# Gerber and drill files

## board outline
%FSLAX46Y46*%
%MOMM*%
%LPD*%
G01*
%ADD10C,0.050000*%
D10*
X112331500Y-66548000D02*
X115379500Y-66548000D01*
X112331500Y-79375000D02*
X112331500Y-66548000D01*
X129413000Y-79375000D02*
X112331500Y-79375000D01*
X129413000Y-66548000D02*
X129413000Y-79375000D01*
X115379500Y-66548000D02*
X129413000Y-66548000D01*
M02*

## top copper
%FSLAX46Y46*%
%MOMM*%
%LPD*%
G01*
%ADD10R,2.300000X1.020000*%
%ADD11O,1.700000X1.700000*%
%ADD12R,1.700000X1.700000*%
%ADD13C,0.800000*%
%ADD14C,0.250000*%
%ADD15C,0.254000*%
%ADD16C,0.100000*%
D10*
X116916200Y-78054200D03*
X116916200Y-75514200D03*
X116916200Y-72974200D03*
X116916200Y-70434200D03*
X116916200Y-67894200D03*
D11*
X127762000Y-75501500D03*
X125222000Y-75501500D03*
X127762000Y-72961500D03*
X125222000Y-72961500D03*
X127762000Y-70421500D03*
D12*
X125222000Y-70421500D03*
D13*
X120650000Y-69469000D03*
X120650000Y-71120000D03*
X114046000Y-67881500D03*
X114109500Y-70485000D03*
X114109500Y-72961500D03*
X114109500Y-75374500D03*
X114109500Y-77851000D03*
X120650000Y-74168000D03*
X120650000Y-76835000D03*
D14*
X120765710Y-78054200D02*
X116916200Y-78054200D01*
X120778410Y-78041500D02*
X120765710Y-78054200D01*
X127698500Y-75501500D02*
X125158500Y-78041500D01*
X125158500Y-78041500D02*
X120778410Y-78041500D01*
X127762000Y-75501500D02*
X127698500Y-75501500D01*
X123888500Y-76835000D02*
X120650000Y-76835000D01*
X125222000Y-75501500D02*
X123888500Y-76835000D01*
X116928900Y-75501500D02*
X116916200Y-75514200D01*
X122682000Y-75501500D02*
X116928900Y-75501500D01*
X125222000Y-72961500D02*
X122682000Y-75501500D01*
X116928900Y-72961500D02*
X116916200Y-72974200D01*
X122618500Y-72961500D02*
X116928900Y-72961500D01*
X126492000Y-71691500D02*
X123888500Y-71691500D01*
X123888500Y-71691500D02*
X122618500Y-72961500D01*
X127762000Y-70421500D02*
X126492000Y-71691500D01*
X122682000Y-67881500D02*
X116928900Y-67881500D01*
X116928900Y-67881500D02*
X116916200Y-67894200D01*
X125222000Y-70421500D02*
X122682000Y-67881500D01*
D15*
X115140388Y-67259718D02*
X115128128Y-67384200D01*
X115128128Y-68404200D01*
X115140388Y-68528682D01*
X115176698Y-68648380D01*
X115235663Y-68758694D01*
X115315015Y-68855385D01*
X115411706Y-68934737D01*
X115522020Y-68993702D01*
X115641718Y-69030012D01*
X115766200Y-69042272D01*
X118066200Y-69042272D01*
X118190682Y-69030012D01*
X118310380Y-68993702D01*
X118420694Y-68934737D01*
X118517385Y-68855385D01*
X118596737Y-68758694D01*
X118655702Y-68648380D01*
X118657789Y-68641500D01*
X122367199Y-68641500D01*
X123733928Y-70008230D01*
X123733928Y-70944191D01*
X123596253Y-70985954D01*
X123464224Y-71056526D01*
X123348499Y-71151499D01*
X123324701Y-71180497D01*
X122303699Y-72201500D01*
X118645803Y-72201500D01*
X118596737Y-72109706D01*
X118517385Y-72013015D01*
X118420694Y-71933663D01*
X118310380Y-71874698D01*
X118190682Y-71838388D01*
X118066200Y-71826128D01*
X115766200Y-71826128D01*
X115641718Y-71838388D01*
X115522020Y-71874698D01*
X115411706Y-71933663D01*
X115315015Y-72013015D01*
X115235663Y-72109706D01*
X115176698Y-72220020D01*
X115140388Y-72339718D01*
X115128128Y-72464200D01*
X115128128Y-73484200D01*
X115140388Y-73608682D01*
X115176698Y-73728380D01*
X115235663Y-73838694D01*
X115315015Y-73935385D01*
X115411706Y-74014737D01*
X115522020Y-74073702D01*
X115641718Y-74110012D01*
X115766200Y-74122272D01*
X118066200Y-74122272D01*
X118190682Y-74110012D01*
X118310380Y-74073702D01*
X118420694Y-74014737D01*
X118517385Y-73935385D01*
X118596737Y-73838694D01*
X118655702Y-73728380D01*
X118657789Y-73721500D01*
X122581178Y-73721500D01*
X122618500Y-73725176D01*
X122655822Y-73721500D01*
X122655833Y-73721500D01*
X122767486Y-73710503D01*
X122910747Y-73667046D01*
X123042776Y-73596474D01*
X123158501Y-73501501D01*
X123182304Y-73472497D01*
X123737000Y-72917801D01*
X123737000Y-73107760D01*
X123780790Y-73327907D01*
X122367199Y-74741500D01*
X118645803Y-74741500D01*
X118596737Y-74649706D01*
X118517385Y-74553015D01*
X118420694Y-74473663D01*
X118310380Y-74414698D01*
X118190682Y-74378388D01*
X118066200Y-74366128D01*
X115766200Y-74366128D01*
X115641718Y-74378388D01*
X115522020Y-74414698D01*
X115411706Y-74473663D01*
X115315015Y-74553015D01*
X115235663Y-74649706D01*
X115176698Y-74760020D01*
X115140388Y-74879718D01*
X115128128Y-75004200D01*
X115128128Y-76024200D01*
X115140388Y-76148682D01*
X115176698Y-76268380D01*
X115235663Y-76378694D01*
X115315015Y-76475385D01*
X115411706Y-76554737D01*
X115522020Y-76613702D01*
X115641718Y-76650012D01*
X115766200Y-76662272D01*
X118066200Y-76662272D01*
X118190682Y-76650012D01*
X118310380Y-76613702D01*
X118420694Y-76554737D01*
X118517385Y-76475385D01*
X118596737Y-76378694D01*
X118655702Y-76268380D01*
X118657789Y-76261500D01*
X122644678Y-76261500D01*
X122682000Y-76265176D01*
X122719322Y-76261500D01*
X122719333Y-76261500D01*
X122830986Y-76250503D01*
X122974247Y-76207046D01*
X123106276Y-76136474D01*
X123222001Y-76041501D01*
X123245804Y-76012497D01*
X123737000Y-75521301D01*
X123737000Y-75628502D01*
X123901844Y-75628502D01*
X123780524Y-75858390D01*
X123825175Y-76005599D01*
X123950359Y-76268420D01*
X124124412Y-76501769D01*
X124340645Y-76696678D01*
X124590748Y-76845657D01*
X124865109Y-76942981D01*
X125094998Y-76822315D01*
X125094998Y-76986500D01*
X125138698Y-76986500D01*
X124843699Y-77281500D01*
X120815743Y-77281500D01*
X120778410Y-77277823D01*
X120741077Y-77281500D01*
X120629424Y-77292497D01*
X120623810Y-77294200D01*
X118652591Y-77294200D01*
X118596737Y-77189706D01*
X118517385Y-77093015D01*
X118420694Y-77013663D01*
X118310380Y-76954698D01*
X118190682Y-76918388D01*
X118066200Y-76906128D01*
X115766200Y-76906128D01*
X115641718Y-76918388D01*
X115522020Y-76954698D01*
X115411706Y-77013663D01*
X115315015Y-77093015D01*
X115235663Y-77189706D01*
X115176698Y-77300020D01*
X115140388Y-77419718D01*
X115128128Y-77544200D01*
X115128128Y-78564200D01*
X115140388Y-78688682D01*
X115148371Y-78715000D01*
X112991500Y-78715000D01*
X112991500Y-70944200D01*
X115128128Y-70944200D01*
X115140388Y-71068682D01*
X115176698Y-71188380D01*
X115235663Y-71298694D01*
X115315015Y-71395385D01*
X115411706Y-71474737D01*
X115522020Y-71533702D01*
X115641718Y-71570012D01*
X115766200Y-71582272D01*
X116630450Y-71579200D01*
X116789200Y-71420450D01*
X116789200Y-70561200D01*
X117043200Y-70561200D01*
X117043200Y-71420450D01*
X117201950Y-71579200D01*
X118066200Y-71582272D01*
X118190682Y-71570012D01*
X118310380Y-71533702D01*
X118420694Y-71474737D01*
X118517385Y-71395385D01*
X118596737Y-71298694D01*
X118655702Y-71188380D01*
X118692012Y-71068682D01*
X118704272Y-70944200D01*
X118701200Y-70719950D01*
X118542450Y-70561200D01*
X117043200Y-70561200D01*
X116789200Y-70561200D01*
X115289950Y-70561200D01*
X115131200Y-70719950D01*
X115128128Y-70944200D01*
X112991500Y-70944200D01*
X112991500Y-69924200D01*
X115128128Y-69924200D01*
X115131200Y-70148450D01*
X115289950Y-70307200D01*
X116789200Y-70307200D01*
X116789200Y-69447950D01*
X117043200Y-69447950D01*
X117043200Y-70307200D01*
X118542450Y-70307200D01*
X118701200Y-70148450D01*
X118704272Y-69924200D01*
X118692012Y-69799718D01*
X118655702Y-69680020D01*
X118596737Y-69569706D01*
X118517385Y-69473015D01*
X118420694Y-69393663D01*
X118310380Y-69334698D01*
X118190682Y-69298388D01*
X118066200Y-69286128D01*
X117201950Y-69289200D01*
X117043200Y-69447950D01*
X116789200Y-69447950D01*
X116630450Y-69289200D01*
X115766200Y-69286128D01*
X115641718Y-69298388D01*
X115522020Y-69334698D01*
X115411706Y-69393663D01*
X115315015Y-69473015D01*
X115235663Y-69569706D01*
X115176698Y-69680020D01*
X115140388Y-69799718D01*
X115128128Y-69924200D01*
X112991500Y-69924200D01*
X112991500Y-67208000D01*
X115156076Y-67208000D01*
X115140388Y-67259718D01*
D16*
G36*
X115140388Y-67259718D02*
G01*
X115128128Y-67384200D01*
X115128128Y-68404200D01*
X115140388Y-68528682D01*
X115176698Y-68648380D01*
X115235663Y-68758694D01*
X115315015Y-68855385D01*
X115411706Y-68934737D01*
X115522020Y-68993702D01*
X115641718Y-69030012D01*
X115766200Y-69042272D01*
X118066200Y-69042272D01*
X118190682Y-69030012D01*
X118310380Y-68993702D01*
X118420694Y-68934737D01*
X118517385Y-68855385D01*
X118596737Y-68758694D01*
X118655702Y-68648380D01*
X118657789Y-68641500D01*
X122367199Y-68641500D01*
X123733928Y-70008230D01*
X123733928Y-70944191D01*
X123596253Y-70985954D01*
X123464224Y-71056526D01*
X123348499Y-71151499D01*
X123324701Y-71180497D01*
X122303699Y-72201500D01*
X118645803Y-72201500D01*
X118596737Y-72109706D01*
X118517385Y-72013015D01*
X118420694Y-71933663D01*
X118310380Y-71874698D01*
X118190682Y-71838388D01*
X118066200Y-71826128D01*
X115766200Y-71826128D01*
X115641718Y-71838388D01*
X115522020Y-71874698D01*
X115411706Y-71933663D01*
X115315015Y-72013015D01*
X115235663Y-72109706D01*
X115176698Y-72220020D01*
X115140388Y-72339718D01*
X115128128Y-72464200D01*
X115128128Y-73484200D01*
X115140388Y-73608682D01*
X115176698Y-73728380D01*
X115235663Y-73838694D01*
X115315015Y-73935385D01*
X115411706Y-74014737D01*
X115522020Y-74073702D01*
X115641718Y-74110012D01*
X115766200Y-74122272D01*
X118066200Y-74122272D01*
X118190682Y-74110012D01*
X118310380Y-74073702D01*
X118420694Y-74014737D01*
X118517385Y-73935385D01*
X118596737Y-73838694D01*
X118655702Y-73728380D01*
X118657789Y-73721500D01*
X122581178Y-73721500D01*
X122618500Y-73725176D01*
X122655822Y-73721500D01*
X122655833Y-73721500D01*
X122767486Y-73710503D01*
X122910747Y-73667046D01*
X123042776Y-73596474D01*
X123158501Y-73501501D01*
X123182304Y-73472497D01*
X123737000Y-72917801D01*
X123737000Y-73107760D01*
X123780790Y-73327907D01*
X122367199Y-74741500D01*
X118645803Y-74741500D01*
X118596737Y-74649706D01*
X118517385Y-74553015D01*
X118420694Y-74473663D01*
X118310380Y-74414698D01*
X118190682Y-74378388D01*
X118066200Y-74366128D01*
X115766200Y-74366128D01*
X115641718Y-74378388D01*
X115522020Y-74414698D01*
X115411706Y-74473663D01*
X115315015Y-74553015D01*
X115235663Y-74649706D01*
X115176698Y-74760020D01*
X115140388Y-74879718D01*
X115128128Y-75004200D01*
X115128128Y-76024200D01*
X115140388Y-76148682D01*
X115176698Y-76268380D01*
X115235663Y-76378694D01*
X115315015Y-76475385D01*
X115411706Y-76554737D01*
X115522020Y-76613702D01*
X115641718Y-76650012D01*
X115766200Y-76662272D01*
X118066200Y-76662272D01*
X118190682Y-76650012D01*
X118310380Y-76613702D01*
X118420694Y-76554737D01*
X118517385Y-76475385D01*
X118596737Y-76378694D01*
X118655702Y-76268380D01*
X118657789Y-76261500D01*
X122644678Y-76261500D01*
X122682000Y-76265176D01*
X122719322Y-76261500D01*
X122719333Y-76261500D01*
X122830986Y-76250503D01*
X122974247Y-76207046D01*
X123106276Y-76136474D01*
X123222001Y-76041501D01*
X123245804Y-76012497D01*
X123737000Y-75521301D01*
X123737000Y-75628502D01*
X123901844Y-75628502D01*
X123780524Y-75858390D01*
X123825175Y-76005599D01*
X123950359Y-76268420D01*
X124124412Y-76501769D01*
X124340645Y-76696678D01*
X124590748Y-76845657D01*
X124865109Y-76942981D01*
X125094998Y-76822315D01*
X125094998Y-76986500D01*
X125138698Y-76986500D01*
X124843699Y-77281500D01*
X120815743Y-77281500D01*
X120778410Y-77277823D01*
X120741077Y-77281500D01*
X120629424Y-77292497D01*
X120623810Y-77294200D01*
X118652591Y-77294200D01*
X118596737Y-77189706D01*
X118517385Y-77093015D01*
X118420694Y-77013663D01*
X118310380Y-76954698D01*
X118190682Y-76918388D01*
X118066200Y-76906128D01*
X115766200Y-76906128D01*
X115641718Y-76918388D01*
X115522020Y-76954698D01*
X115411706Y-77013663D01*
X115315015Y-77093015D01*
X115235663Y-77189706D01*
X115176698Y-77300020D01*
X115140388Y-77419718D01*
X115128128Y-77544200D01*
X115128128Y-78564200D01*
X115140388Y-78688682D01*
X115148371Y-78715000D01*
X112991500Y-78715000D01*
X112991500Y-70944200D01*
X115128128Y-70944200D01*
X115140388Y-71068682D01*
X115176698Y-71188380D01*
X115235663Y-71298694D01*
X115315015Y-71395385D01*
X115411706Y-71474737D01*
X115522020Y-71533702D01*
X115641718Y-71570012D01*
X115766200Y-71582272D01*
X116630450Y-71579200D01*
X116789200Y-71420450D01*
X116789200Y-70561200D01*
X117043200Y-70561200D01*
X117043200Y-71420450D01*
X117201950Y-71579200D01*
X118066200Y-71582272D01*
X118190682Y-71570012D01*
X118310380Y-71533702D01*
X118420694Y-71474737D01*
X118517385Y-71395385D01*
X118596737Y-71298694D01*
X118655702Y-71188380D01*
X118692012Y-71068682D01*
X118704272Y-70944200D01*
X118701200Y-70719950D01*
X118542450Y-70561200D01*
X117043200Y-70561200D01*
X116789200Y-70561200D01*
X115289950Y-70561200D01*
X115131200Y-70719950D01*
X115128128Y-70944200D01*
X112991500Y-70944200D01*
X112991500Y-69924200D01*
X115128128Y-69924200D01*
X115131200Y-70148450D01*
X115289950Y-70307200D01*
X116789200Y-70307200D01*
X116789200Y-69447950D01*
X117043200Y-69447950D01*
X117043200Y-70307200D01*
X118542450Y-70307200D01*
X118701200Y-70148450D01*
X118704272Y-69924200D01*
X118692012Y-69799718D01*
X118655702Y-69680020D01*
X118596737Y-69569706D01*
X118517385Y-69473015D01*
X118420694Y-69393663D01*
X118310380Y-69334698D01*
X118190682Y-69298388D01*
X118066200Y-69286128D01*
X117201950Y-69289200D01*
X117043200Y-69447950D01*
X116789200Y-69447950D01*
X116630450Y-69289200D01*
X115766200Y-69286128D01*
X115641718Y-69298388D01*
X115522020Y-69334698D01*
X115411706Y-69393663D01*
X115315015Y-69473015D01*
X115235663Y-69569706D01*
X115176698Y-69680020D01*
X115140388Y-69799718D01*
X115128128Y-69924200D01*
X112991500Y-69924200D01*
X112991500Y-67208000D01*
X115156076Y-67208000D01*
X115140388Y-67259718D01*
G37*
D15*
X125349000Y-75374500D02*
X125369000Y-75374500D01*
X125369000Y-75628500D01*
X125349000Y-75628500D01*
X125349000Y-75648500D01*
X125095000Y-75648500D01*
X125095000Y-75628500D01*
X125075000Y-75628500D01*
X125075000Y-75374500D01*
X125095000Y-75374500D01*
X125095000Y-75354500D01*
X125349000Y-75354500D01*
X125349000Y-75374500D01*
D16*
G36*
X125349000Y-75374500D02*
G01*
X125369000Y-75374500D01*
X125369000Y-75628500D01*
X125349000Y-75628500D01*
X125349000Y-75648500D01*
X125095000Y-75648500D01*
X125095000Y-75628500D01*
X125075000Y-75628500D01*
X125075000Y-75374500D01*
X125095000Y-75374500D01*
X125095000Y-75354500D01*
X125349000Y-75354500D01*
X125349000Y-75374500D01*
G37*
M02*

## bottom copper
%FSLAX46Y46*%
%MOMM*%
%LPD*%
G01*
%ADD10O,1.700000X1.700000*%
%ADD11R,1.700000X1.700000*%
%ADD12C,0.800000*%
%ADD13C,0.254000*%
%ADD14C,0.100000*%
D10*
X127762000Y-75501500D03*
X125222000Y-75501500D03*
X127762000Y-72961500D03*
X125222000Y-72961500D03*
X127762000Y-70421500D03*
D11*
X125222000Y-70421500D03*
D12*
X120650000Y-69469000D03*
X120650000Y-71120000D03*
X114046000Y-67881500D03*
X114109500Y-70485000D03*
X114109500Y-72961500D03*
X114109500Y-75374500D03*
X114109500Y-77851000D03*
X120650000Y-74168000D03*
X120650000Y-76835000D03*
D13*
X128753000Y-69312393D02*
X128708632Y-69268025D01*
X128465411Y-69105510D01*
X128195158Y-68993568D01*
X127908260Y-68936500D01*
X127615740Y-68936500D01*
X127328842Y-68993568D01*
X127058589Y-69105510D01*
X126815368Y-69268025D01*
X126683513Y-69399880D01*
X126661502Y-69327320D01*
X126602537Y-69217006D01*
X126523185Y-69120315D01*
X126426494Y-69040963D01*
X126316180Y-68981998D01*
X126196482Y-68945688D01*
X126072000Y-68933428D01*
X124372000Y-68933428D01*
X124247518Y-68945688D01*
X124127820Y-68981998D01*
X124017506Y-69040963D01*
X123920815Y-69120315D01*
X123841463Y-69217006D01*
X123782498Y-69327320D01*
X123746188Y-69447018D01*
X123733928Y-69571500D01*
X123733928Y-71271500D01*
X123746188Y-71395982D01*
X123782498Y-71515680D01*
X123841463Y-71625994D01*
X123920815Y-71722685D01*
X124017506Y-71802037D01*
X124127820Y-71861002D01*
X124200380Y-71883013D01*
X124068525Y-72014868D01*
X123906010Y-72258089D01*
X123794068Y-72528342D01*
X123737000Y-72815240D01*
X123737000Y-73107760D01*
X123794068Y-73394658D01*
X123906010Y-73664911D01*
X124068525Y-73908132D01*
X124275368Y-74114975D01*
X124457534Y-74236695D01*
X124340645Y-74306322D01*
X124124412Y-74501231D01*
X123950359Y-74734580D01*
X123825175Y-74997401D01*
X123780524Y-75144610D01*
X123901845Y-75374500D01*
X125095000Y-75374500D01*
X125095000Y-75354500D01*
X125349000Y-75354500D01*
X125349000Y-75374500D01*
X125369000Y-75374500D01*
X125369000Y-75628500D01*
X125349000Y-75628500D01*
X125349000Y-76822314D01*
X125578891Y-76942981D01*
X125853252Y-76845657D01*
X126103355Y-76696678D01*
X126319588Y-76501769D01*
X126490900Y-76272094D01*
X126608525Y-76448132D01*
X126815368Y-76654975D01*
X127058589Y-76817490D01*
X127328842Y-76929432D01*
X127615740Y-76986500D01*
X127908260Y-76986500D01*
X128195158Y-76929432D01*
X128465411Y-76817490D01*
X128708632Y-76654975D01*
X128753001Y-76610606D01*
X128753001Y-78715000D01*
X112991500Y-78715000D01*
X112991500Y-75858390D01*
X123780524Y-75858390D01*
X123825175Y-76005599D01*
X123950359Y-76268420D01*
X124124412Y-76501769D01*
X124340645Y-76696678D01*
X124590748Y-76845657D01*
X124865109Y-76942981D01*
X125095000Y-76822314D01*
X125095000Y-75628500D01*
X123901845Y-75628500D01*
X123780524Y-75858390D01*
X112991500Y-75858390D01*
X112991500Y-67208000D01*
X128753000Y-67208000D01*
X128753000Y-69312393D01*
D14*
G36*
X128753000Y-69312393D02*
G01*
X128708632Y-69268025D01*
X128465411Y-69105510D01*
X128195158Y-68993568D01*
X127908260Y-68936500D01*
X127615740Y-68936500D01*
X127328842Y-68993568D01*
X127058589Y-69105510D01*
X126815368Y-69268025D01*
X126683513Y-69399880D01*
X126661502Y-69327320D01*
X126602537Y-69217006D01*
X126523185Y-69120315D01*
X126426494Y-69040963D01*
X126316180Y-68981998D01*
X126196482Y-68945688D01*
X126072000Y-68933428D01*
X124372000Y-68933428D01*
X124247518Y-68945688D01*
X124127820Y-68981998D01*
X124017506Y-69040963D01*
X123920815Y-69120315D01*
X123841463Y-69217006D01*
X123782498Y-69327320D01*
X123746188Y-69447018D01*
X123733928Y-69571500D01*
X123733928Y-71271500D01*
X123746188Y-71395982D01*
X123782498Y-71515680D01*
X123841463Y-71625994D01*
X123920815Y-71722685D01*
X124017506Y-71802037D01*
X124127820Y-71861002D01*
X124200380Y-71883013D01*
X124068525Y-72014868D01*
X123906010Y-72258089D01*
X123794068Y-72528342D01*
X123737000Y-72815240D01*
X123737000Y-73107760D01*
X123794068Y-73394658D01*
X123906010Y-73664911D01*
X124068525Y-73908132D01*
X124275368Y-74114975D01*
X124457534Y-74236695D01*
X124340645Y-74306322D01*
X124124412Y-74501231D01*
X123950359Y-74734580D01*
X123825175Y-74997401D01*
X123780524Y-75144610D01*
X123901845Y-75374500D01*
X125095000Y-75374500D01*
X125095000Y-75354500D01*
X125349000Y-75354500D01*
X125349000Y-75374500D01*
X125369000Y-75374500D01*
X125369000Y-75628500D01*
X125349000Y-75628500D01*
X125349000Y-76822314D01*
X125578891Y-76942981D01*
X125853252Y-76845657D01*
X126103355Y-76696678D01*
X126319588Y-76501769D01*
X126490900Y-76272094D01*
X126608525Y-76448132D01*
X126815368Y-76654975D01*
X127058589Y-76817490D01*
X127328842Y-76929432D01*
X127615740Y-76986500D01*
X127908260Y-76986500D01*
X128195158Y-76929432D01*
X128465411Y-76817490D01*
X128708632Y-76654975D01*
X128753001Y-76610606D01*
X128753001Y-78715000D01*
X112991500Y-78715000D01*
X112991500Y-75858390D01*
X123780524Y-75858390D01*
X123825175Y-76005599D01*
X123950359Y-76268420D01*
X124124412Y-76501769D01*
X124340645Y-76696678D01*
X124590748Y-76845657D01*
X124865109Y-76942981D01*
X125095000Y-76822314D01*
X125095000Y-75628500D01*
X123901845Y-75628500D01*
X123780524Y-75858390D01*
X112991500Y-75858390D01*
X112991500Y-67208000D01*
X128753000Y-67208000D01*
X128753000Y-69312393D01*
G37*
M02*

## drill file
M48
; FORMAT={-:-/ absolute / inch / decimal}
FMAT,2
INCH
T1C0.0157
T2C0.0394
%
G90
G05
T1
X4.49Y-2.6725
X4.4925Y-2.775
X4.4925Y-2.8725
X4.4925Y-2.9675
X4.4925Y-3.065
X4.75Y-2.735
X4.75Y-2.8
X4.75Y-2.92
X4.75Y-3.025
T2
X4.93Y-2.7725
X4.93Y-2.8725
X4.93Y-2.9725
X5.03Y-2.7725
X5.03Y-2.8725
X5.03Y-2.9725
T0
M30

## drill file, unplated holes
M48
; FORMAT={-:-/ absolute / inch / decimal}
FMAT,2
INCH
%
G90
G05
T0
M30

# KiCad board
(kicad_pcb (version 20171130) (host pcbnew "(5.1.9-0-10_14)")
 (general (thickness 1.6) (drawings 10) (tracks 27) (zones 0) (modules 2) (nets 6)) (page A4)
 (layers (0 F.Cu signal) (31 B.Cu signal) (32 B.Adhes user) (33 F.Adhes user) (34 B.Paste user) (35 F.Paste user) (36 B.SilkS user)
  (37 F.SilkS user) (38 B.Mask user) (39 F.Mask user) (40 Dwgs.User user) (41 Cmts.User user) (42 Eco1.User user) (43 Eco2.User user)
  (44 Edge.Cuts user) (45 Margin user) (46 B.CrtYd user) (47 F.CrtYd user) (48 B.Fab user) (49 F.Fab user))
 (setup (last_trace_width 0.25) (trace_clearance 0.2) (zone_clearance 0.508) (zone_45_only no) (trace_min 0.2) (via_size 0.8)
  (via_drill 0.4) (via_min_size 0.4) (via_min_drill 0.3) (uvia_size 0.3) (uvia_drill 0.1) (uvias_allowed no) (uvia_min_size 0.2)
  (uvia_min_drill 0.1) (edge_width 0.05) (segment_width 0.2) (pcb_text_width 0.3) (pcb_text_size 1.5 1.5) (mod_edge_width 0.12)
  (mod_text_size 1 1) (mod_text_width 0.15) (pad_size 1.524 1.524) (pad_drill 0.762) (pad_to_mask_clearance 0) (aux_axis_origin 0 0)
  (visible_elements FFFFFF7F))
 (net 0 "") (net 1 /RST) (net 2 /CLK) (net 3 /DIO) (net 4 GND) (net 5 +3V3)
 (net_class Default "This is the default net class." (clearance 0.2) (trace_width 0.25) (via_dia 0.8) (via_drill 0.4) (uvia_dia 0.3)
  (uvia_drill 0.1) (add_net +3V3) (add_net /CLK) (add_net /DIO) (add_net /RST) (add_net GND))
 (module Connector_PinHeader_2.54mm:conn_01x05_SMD (layer F.Cu) (at 116.967 65.659)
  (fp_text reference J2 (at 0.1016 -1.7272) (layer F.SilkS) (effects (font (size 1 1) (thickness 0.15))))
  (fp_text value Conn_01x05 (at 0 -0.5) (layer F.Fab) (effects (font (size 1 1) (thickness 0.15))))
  (pad 5 smd rect (at -0.0508 12.3952 90) (size 1.02 2.3) (layers F.Cu F.Paste F.Mask) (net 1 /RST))
  (pad 4 smd rect (at -0.0508 9.8552 90) (size 1.02 2.3) (layers F.Cu F.Paste F.Mask) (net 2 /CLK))
  (pad 3 smd rect (at -0.0508 7.3152 90) (size 1.02 2.3) (layers F.Cu F.Paste F.Mask) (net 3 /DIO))
  (pad 2 smd rect (at -0.0508 4.7752 90) (size 1.02 2.3) (layers F.Cu F.Paste F.Mask) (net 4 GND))
  (pad 1 smd rect (at -0.0508 2.2352 90) (size 1.02 2.3) (layers F.Cu F.Paste F.Mask) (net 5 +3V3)))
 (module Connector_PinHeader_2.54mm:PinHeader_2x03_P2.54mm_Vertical (layer F.Cu) (at 125.222 70.4215)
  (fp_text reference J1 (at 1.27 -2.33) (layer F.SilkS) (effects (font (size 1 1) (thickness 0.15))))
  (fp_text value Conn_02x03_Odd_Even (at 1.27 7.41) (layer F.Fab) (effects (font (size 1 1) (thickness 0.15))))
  (pad 6 thru_hole oval (at 2.54 5.08) (size 1.7 1.7) (drill 1) (layers *.Cu *.Mask) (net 1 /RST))
  (pad 5 thru_hole oval (at 0 5.08) (size 1.7 1.7) (drill 1) (layers *.Cu *.Mask) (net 4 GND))
  (pad 4 thru_hole oval (at 2.54 2.54) (size 1.7 1.7) (drill 1) (layers *.Cu *.Mask))
  (pad 3 thru_hole oval (at 0 2.54) (size 1.7 1.7) (drill 1) (layers *.Cu *.Mask) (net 2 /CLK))
  (pad 2 thru_hole oval (at 2.54 0) (size 1.7 1.7) (drill 1) (layers *.Cu *.Mask) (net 3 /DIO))
  (pad 1 thru_hole rect (at 0 0) (size 1.7 1.7) (drill 1) (layers *.Cu *.Mask) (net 5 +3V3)))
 (gr_line (start 112.3315 66.548) (end 115.3795 66.548) (layer Edge.Cuts) (width 0.05))
 (gr_line (start 112.3315 79.375) (end 112.3315 66.548) (layer Edge.Cuts) (width 0.05))
 (gr_line (start 129.413 79.375) (end 112.3315 79.375) (layer Edge.Cuts) (width 0.05))
 (gr_line (start 129.413 66.548) (end 129.413 79.375) (layer Edge.Cuts) (width 0.05))
 (gr_line (start 115.3795 66.548) (end 129.413 66.548) (layer Edge.Cuts) (width 0.05))
 (segment (start 120.76571 78.0542) (end 116.9162 78.0542) (width 0.25) (layer F.Cu) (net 1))
 (segment (start 120.77841 78.0415) (end 120.76571 78.0542) (width 0.25) (layer F.Cu) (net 1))
 (segment (start 127.6985 75.5015) (end 125.1585 78.0415) (width 0.25) (layer F.Cu) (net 1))
 (segment (start 125.1585 78.0415) (end 120.77841 78.0415) (width 0.25) (layer F.Cu) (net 1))
 (segment (start 127.762 75.5015) (end 127.6985 75.5015) (width 0.25) (layer F.Cu) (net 1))
 (via (at 120.65 69.469) (size 0.8) (drill 0.4) (layers F.Cu B.Cu) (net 4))
 (via (at 120.65 71.12) (size 0.8) (drill 0.4) (layers F.Cu B.Cu) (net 4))
 (via (at 114.046 67.8815) (size 0.8) (drill 0.4) (layers F.Cu B.Cu) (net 4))
 (via (at 114.1095 70.485) (size 0.8) (drill 0.4) (layers F.Cu B.Cu) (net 4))
 (via (at 114.1095 72.9615) (size 0.8) (drill 0.4) (layers F.Cu B.Cu) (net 4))
 (via (at 114.1095 75.3745) (size 0.8) (drill 0.4) (layers F.Cu B.Cu) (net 4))
 (via (at 114.1095 77.851) (size 0.8) (drill 0.4) (layers F.Cu B.Cu) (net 4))
 (via (at 120.65 74.168) (size 0.8) (drill 0.4) (layers F.Cu B.Cu) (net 4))
 (via (at 120.65 76.835) (size 0.8) (drill 0.4) (layers F.Cu B.Cu) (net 4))
 (segment (start 123.8885 76.835) (end 120.65 76.835) (width 0.25) (layer F.Cu) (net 4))
 (segment (start 125.222 75.5015) (end 123.8885 76.835) (width 0.25) (layer F.Cu) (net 4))
 (segment (start 116.9289 75.5015) (end 116.9162 75.5142) (width 0.25) (layer F.Cu) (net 2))
 (segment (start 122.682 75.5015) (end 116.9289 75.5015) (width 0.25) (layer F.Cu) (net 2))
 (segment (start 125.222 72.9615) (end 122.682 75.5015) (width 0.25) (layer F.Cu) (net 2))
 (segment (start 116.9289 72.9615) (end 116.9162 72.9742) (width 0.25) (layer F.Cu) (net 3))
 (segment (start 122.6185 72.9615) (end 116.9289 72.9615) (width 0.25) (layer F.Cu) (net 3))
 (segment (start 126.492 71.6915) (end 123.8885 71.6915) (width 0.25) (layer F.Cu) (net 3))
 (segment (start 123.8885 71.6915) (end 122.6185 72.9615) (width 0.25) (layer F.Cu) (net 3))
 (segment (start 127.762 70.4215) (end 126.492 71.6915) (width 0.25) (layer F.Cu) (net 3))
 (segment (start 122.682 67.8815) (end 116.9289 67.8815) (width 0.25) (layer F.Cu) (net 5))
 (segment (start 116.9289 67.8815) (end 116.9162 67.8942) (width 0.25) (layer F.Cu) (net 5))
 (segment (start 125.222 70.4215) (end 122.682 67.8815) (width 0.25) (layer F.Cu) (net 5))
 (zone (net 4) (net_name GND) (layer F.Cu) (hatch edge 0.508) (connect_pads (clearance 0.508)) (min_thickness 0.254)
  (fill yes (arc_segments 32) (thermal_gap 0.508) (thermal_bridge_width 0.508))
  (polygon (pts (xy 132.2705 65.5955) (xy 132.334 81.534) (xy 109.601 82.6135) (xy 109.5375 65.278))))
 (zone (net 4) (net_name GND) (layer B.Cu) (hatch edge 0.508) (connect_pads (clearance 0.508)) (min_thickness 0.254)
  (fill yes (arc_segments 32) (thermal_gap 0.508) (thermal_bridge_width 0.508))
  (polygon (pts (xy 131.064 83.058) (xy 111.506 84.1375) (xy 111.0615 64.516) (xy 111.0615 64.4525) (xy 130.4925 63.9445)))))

